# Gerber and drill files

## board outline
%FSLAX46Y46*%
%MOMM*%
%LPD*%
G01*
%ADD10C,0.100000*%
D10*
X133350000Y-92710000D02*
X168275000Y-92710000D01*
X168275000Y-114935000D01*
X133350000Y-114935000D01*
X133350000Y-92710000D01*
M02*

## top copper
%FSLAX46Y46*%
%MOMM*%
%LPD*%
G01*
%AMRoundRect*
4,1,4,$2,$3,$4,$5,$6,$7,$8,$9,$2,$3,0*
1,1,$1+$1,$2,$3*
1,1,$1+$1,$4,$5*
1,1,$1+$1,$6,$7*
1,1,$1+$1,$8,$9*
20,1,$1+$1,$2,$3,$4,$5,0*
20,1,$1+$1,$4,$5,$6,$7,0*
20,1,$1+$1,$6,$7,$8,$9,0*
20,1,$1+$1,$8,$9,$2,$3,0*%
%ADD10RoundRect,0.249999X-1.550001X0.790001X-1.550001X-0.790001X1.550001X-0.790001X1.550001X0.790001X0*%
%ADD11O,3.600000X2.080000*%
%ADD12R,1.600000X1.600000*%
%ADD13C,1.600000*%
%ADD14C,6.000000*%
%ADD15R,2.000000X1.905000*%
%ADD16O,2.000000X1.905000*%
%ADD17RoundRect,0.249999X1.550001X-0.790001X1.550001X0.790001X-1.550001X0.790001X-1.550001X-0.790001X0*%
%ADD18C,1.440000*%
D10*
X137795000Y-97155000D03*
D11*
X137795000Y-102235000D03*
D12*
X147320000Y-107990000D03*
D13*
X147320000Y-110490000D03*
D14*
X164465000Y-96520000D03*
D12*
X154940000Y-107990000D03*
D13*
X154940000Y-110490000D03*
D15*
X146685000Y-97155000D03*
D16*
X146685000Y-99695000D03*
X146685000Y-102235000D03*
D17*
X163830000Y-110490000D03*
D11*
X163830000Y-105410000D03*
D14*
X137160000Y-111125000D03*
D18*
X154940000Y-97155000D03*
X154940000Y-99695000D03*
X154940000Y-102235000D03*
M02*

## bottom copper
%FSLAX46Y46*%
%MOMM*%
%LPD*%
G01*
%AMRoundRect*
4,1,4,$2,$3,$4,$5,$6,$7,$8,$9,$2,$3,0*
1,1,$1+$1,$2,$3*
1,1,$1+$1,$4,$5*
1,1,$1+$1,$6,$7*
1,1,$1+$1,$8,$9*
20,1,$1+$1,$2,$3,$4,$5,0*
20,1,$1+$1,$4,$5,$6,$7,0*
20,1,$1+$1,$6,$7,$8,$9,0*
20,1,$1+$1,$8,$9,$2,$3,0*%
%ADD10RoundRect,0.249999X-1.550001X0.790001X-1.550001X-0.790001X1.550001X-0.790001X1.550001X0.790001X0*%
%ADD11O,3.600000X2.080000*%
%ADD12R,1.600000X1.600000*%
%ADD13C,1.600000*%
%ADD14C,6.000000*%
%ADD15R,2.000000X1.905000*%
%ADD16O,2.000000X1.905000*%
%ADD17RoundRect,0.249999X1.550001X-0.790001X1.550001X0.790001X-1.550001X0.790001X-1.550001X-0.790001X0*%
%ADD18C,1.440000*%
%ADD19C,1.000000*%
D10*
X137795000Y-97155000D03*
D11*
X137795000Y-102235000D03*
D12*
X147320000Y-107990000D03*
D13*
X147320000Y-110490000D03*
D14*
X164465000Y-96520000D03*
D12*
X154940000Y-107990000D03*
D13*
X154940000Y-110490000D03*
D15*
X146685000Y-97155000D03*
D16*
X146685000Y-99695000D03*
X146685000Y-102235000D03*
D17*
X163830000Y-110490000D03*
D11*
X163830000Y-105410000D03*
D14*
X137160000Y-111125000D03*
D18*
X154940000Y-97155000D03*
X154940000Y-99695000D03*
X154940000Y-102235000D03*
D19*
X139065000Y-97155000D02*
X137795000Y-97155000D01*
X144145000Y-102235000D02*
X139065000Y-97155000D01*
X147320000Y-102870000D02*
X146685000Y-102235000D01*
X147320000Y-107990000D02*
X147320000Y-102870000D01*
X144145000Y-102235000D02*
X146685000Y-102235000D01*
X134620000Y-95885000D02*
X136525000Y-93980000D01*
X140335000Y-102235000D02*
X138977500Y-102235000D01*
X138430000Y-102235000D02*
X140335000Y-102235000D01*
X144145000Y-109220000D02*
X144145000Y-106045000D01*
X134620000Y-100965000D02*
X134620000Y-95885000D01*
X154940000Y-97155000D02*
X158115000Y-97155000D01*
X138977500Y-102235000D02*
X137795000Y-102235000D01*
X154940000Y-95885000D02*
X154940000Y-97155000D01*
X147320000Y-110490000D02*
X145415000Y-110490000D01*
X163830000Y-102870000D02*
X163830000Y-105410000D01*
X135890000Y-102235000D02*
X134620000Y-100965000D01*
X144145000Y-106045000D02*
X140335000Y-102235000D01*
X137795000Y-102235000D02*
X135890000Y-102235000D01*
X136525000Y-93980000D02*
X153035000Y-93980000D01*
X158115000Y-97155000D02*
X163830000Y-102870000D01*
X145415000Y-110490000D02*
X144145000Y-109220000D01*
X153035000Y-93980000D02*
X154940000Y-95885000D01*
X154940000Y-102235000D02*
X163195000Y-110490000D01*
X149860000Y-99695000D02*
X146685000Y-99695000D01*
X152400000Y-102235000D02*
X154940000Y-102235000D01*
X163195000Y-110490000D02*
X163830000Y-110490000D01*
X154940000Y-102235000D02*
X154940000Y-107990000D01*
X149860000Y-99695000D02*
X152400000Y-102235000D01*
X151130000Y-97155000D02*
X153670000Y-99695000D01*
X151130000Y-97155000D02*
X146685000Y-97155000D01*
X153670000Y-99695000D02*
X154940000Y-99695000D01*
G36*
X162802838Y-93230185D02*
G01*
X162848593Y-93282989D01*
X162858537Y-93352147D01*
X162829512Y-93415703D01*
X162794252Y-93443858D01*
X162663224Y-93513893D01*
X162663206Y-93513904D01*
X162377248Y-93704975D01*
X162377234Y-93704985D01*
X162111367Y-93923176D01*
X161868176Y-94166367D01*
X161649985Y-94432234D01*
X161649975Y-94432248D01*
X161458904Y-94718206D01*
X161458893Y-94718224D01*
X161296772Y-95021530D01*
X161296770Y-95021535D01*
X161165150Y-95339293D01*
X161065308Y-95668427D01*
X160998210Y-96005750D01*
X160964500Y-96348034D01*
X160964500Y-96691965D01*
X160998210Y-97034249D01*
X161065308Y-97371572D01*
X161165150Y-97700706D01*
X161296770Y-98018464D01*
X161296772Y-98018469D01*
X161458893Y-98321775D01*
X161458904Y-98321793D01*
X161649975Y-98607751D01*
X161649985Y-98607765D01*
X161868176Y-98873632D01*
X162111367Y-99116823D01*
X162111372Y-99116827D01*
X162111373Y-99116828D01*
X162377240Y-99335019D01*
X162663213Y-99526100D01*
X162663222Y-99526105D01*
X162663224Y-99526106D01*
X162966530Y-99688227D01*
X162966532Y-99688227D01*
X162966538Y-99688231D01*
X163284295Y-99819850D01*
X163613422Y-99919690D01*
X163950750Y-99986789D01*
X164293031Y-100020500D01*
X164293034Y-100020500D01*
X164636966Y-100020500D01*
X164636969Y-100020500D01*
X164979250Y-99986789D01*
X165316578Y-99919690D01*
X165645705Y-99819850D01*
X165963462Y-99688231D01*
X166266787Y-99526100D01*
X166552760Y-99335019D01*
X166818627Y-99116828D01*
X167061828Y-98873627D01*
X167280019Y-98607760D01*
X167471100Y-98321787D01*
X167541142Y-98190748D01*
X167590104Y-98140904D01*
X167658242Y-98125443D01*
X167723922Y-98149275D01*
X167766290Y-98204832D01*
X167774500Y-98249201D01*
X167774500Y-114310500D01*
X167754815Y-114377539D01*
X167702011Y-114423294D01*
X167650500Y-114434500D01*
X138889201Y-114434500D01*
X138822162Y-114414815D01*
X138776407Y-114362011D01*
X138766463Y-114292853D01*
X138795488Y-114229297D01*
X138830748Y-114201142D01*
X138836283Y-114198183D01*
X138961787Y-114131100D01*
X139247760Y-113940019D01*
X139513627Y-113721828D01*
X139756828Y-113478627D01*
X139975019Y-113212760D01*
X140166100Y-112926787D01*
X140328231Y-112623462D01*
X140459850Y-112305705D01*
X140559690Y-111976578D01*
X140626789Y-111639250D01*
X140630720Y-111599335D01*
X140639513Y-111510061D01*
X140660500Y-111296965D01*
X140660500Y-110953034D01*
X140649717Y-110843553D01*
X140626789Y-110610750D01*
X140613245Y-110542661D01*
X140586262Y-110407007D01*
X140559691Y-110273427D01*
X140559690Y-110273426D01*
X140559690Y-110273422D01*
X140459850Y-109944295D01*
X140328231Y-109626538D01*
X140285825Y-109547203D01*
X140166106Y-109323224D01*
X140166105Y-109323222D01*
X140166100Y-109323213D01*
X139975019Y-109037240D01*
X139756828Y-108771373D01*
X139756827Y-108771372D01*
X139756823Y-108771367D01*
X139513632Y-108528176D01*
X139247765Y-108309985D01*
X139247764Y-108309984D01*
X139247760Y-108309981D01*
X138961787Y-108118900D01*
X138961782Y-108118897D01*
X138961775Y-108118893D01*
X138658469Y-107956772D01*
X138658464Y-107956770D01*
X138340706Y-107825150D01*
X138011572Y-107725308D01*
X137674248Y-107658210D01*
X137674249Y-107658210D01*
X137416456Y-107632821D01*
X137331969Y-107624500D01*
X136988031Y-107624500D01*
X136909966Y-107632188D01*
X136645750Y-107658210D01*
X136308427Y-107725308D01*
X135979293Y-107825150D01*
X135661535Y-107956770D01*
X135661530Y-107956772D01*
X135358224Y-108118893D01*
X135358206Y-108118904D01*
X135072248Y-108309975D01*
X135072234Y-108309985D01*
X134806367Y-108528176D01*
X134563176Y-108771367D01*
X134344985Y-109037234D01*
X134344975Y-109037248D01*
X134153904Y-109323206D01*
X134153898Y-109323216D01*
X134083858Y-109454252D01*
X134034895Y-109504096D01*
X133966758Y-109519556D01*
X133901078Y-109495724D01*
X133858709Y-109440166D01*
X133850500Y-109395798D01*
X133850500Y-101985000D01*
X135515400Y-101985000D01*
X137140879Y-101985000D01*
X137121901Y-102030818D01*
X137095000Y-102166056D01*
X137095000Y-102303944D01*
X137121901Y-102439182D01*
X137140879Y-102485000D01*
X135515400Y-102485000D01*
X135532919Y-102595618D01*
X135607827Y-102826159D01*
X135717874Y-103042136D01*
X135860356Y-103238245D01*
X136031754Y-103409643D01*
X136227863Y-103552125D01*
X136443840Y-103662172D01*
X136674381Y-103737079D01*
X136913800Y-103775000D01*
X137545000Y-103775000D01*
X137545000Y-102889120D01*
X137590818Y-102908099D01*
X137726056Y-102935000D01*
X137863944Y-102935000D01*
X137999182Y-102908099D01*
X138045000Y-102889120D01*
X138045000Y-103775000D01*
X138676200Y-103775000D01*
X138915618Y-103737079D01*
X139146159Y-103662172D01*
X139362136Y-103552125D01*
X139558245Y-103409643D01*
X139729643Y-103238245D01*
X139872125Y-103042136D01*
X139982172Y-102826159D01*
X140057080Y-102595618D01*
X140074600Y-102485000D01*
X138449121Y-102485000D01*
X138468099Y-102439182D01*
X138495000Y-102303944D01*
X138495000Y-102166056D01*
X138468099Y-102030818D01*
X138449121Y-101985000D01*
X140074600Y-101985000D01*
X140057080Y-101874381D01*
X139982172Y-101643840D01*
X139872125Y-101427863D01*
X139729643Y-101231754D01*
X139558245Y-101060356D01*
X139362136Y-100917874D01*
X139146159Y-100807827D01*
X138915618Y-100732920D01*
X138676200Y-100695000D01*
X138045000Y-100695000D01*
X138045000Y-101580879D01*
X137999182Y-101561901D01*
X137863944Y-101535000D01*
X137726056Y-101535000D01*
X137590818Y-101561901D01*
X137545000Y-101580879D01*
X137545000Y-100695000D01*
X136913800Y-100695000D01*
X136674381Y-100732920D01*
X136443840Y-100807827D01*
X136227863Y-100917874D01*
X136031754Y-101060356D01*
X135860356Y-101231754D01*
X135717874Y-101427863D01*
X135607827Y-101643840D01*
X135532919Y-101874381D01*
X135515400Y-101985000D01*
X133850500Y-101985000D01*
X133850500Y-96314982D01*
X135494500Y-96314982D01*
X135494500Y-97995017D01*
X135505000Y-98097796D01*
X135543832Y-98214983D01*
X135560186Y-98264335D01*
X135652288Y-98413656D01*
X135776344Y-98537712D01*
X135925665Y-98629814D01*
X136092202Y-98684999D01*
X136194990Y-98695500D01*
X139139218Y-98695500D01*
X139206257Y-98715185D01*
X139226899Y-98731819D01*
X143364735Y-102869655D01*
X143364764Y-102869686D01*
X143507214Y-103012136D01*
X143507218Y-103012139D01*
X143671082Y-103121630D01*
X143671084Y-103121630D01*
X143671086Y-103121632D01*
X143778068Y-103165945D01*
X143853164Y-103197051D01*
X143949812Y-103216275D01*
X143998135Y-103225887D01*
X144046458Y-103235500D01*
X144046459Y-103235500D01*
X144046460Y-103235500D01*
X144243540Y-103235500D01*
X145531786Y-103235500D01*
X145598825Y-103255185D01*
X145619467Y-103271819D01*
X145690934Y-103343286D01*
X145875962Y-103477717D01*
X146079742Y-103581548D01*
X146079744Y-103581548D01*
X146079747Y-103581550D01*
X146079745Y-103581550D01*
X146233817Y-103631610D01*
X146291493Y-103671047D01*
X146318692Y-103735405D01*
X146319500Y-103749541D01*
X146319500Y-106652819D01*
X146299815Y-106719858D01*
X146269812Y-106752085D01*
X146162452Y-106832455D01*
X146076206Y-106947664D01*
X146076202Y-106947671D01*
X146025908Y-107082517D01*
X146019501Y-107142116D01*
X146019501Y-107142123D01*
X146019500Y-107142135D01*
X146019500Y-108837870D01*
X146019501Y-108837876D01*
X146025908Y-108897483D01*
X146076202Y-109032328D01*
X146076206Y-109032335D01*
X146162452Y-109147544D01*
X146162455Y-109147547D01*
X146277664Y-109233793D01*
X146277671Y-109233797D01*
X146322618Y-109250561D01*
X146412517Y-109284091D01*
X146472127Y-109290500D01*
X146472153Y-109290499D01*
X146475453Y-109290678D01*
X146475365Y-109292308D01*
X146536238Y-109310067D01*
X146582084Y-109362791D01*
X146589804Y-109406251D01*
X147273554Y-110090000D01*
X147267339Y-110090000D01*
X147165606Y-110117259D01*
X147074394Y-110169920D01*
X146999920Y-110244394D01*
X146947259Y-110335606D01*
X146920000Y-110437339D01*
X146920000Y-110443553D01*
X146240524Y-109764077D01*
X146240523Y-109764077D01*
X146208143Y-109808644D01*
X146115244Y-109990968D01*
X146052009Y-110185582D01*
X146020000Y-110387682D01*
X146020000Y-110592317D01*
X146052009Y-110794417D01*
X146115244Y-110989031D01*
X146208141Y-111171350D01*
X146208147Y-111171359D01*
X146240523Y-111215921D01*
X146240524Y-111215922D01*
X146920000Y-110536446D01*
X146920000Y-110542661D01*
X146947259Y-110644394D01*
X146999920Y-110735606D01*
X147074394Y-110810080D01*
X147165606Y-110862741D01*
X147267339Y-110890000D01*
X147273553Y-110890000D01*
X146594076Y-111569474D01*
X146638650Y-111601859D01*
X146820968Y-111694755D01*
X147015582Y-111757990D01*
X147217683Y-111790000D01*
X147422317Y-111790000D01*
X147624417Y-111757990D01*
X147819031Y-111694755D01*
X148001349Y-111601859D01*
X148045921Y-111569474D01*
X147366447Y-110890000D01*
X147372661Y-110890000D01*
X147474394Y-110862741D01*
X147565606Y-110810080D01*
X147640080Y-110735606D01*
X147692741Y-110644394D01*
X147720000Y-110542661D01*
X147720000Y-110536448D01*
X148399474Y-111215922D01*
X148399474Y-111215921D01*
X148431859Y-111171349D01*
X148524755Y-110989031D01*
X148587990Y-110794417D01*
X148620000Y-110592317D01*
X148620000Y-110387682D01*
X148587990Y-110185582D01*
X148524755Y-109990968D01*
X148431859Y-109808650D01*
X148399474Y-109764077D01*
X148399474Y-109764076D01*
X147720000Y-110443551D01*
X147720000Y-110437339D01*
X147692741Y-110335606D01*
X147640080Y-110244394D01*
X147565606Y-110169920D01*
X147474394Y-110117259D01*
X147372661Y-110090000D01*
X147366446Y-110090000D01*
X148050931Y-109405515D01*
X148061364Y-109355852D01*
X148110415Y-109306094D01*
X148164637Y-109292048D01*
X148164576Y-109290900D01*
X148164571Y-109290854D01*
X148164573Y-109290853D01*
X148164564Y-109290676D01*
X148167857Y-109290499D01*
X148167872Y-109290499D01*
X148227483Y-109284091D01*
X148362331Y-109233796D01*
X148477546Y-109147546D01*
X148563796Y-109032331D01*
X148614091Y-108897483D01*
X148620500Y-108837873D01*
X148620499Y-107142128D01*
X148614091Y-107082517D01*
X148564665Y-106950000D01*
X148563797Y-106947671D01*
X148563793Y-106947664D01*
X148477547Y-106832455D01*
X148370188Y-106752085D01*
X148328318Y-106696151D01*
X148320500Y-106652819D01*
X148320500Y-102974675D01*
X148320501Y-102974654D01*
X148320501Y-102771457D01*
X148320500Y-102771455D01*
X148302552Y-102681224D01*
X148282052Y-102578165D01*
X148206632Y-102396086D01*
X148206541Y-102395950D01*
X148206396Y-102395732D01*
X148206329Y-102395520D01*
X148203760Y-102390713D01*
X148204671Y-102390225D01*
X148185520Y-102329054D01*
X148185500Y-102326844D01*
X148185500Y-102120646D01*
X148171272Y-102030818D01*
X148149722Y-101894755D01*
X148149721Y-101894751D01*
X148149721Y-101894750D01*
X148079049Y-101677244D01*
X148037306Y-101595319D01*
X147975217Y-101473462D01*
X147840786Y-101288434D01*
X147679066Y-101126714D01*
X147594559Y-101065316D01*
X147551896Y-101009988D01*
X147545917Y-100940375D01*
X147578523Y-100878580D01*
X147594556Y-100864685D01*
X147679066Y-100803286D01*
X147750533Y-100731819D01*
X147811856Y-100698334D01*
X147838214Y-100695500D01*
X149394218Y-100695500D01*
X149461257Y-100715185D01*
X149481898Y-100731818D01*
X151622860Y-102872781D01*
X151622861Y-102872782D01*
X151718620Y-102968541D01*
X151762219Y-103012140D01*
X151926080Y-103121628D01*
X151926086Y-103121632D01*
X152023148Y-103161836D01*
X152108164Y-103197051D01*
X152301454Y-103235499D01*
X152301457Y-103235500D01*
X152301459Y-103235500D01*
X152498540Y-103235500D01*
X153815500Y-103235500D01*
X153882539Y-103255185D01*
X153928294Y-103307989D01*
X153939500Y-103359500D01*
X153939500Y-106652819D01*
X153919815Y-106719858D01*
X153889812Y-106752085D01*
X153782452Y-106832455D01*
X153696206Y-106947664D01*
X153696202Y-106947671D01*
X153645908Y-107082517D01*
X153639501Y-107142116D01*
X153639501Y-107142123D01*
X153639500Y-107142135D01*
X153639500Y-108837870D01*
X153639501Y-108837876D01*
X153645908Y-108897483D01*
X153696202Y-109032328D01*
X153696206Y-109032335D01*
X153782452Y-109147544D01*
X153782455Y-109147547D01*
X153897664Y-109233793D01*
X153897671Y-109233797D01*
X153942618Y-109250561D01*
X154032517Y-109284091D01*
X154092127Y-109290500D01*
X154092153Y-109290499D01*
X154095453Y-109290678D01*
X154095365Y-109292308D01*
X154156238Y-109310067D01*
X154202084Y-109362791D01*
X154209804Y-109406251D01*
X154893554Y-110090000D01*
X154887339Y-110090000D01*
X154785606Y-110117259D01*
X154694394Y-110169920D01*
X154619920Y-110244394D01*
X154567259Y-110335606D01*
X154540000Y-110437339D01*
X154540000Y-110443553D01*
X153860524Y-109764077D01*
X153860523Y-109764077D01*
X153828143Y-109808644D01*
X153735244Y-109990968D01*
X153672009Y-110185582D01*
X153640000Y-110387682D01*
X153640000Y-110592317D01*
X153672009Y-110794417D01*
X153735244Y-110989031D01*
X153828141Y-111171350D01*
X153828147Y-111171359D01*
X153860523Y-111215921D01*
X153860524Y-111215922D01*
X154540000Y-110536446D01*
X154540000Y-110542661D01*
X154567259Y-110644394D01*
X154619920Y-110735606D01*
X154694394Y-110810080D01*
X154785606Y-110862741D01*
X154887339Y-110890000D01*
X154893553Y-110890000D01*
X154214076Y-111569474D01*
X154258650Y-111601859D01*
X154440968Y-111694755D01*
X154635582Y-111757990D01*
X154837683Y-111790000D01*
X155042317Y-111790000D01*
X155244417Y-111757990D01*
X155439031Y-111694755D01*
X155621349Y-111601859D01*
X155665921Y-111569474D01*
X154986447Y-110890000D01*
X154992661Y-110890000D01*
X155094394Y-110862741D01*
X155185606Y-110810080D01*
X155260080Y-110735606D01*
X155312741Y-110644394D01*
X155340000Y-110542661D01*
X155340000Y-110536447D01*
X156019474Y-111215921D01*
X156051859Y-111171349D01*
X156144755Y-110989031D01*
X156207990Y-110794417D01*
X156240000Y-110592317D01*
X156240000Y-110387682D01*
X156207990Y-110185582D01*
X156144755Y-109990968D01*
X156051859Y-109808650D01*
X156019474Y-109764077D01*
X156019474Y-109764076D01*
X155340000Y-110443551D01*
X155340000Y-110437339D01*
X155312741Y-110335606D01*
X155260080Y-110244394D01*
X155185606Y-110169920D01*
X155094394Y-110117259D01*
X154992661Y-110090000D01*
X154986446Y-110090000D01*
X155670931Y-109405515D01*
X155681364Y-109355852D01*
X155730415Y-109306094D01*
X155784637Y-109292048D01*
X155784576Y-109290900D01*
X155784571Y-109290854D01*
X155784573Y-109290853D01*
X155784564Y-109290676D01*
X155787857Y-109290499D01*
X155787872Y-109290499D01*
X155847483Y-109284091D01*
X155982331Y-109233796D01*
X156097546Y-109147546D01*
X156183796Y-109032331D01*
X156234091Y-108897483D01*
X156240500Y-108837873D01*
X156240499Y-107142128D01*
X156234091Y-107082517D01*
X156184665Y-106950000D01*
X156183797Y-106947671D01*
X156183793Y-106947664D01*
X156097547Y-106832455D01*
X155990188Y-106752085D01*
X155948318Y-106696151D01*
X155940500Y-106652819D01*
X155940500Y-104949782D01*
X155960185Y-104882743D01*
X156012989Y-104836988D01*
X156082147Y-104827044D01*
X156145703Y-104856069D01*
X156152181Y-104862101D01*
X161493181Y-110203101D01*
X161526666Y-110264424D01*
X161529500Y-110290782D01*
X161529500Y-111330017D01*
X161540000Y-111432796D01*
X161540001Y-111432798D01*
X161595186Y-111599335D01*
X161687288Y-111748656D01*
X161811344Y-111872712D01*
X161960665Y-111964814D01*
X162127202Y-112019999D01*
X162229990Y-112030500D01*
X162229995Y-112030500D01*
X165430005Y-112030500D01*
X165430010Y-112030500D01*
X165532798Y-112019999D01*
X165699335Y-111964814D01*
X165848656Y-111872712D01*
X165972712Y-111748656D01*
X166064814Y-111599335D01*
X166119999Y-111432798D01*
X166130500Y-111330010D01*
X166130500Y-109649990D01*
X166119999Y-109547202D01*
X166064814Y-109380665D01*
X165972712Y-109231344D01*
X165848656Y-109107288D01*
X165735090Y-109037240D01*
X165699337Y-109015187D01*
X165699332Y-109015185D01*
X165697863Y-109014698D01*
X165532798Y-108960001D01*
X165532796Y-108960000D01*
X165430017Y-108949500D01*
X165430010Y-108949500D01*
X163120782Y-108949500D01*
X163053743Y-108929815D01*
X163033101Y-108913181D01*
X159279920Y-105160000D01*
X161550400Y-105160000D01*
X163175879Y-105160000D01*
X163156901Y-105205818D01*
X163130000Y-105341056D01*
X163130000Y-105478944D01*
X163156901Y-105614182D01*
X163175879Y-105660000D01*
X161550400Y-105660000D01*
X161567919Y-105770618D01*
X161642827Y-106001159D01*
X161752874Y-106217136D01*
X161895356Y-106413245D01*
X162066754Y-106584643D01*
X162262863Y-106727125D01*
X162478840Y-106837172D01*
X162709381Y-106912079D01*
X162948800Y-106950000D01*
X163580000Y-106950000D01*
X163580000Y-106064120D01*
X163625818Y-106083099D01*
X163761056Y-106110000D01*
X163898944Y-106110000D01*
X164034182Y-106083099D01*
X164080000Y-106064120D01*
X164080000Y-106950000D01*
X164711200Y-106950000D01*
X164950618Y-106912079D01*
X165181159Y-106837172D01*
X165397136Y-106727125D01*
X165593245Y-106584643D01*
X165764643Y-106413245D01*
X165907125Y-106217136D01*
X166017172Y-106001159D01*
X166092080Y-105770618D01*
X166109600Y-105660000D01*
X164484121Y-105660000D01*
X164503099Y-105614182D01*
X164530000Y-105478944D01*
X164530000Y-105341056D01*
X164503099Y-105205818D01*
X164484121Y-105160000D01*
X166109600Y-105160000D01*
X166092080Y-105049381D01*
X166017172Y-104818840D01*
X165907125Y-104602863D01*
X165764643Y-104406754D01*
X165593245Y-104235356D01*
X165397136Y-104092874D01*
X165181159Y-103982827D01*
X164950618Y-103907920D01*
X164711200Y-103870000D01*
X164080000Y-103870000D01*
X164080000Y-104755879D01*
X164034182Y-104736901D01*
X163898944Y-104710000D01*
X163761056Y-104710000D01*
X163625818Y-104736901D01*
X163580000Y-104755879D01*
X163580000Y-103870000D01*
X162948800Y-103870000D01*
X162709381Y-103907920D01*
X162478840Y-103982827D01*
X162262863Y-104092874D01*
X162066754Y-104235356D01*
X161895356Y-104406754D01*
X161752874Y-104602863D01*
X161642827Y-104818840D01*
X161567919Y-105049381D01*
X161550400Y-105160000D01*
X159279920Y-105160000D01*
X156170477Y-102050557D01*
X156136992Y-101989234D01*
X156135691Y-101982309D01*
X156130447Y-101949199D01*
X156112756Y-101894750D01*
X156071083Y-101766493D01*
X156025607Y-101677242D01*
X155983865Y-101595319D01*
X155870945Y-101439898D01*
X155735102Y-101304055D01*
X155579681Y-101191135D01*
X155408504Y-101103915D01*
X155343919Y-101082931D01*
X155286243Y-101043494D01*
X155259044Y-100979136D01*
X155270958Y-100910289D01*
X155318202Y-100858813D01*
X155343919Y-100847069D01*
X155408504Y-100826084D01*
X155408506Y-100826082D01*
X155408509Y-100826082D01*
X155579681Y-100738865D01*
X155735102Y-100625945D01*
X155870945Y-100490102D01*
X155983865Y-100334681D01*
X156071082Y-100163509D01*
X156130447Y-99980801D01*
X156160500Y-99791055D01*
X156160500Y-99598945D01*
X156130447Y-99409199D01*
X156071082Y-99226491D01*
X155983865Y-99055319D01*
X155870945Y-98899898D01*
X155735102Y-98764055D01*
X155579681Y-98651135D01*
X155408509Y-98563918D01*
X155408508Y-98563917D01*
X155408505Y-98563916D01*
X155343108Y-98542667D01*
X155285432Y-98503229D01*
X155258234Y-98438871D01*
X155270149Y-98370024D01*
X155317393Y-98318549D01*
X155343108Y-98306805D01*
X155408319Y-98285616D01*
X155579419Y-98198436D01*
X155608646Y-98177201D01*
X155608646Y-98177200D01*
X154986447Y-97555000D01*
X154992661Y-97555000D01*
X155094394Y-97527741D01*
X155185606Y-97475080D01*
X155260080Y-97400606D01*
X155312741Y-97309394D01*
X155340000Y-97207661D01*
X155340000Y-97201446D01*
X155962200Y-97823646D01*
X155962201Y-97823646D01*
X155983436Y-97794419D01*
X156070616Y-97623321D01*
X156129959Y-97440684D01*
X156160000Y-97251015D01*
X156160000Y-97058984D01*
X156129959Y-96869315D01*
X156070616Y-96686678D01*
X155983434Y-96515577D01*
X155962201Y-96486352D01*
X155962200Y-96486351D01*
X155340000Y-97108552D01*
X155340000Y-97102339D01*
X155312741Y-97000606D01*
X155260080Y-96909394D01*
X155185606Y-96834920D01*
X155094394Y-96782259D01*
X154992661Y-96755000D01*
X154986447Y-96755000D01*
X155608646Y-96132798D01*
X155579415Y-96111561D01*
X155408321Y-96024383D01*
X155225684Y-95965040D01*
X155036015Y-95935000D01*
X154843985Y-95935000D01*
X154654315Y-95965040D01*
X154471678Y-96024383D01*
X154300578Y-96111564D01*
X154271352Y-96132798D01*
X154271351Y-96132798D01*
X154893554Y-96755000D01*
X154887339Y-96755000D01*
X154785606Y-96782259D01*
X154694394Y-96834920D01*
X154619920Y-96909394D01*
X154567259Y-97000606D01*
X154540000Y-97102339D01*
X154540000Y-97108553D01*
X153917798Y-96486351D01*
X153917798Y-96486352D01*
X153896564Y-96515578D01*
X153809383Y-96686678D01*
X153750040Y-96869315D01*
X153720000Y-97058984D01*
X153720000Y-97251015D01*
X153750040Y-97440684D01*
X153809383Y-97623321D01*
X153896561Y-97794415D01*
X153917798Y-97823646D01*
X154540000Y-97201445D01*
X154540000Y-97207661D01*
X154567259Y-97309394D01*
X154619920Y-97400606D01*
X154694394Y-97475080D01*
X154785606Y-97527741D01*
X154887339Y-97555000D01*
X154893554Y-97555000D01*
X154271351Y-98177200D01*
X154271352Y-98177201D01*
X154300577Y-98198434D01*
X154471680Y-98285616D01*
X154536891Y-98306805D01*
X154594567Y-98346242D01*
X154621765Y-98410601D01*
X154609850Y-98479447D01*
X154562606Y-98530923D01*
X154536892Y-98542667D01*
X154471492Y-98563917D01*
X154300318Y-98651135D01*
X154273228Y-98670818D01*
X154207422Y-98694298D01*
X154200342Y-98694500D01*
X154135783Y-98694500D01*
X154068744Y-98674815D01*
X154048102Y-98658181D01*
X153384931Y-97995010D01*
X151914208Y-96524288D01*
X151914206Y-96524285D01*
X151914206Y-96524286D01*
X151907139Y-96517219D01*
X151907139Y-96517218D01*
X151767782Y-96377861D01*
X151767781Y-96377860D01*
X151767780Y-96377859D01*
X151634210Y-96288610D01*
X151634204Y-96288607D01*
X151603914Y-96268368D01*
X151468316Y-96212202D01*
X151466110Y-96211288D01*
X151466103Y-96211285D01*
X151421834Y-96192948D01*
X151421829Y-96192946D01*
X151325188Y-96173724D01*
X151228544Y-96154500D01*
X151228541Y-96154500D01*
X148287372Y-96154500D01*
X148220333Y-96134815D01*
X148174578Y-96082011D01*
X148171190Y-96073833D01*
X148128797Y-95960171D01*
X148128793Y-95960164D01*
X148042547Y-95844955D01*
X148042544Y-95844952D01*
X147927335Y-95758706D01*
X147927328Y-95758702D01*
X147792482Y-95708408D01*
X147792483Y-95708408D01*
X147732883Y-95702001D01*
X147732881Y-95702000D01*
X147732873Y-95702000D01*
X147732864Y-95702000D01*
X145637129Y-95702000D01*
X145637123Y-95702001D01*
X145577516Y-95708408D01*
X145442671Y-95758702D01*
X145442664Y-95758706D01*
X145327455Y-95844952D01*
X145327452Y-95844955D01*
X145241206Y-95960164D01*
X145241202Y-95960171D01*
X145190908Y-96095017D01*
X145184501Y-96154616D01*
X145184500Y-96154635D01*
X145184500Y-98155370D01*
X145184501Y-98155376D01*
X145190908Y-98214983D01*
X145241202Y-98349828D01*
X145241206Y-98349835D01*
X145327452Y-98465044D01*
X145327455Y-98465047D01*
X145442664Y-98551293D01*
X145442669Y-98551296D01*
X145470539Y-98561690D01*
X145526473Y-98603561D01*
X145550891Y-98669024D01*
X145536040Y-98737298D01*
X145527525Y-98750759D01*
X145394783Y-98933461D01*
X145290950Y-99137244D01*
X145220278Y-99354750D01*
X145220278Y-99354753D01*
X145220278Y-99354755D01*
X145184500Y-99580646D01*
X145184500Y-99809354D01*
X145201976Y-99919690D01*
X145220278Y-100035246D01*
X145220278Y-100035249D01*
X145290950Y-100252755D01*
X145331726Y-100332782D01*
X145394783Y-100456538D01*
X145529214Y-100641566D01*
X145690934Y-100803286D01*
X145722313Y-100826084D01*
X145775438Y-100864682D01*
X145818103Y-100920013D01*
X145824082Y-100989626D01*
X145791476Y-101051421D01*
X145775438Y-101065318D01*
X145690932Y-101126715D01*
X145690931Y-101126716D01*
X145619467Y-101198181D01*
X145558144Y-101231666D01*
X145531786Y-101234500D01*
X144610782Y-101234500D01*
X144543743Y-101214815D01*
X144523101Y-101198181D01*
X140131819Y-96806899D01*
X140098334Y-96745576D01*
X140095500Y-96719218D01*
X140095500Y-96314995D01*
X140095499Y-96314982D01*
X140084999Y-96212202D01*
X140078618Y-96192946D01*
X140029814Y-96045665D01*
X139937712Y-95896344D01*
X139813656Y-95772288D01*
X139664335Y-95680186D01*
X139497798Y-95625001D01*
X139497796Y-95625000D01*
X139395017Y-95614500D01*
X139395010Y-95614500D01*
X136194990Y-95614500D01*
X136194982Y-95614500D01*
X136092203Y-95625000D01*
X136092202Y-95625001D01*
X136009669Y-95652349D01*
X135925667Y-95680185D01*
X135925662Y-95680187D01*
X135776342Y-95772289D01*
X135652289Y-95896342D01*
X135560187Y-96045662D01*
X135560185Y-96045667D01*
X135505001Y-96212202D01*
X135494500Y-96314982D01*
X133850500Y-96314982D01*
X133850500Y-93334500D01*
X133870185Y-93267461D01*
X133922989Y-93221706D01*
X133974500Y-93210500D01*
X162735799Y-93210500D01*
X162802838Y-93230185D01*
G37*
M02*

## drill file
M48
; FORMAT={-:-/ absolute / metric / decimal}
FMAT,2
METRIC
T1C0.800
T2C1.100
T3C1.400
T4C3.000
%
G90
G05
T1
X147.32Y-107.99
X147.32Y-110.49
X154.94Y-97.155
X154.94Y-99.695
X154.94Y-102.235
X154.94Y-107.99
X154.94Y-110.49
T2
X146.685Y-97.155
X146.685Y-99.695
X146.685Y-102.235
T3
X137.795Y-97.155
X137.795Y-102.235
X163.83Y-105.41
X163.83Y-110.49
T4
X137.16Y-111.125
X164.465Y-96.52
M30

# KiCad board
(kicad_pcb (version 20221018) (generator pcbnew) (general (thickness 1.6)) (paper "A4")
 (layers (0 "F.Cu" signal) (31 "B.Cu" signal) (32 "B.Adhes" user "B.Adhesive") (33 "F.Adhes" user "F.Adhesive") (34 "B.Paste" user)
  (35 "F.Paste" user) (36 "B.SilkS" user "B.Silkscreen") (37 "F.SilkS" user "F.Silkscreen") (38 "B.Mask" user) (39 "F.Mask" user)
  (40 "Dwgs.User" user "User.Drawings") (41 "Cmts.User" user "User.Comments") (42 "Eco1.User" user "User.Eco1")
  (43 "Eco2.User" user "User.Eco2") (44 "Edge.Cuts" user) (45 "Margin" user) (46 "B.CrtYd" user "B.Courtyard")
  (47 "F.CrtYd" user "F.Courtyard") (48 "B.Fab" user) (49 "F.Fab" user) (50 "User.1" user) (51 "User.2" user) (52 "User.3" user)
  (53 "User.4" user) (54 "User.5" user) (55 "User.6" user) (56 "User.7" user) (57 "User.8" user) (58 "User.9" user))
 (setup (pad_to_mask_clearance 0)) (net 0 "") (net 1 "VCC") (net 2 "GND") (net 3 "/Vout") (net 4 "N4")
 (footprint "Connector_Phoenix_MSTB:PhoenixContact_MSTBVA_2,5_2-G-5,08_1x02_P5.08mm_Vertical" (layer "F.Cu") (at 137.795 97.155 -90)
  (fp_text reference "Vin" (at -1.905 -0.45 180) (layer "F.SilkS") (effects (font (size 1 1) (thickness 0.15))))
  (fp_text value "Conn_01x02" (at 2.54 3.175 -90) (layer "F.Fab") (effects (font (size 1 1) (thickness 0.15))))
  (pad "1" thru_hole roundrect (at 0 0 270) (size 2.08 3.6) (drill 1.4) (layers "*.Cu" "*.Mask") (roundrect_rratio 0.1201918269)
   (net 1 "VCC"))
  (pad "2" thru_hole oval (at 5.08 0 270) (size 2.08 3.6) (drill 1.4) (layers "*.Cu" "*.Mask") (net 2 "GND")))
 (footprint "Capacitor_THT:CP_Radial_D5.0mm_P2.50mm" (layer "F.Cu") (at 147.32 107.99 -90)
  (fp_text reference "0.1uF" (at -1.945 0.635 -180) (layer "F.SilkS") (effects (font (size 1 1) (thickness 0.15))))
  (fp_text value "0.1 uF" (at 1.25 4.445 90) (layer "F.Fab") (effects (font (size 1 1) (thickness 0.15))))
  (pad "1" thru_hole rect (at 0 0 270) (size 1.6 1.6) (drill 0.8) (layers "*.Cu" "*.Mask") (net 1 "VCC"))
  (pad "2" thru_hole circle (at 2.5 0 270) (size 1.6 1.6) (drill 0.8) (layers "*.Cu" "*.Mask") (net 2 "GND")))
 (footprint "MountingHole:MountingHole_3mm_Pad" (layer "F.Cu") (at 164.465 96.52)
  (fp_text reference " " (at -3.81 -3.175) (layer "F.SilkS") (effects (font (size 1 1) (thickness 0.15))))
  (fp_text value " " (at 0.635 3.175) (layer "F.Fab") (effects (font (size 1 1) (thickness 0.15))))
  (pad "1" thru_hole circle (at 0 0) (size 6 6) (drill 3) (layers "*.Cu" "*.Mask")))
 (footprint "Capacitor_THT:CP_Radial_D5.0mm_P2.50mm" (layer "F.Cu") (at 154.94 107.99 -90)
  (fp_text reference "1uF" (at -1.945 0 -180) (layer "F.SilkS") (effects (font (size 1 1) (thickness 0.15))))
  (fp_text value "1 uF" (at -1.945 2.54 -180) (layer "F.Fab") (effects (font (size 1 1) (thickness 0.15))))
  (pad "1" thru_hole rect (at 0 0 270) (size 1.6 1.6) (drill 0.8) (layers "*.Cu" "*.Mask") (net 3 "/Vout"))
  (pad "2" thru_hole circle (at 2.5 0 270) (size 1.6 1.6) (drill 0.8) (layers "*.Cu" "*.Mask") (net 2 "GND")))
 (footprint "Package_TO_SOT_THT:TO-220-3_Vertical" (layer "F.Cu") (at 146.685 97.155 -90)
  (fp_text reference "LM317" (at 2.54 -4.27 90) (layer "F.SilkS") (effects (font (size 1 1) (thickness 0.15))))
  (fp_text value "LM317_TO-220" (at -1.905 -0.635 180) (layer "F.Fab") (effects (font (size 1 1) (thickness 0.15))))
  (pad "1" thru_hole rect (at 0 0 270) (size 1.905 2) (drill 1.1) (layers "*.Cu" "*.Mask") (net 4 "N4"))
  (pad "2" thru_hole oval (at 2.54 0 270) (size 1.905 2) (drill 1.1) (layers "*.Cu" "*.Mask") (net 3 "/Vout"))
  (pad "3" thru_hole oval (at 5.08 0 270) (size 1.905 2) (drill 1.1) (layers "*.Cu" "*.Mask") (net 1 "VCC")))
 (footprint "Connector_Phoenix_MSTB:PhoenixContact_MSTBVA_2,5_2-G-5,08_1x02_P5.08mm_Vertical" (layer "F.Cu") (at 163.83 110.49 90)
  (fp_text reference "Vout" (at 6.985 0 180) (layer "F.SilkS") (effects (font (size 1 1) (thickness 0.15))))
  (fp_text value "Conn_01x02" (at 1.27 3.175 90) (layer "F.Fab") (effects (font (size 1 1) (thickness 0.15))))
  (pad "1" thru_hole roundrect (at 0 0 90) (size 2.08 3.6) (drill 1.4) (layers "*.Cu" "*.Mask") (roundrect_rratio 0.1201918269)
   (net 3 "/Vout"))
  (pad "2" thru_hole oval (at 5.08 0 90) (size 2.08 3.6) (drill 1.4) (layers "*.Cu" "*.Mask") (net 2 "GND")))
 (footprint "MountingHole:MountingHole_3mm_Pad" (layer "F.Cu") (at 137.16 111.125)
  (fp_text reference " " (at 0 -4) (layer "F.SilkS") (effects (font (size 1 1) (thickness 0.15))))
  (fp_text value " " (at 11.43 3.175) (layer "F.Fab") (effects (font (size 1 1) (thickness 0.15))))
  (pad "1" thru_hole circle (at 0 0) (size 6 6) (drill 3) (layers "*.Cu" "*.Mask")))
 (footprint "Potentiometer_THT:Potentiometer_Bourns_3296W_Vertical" (layer "F.Cu") (at 154.94 97.155 90)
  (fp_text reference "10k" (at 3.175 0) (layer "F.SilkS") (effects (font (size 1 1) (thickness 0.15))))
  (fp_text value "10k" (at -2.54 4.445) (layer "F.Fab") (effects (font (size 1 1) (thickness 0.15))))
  (pad "1" thru_hole circle (at 0 0 90) (size 1.44 1.44) (drill 0.8) (layers "*.Cu" "*.Mask") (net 2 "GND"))
  (pad "2" thru_hole circle (at -2.54 0 90) (size 1.44 1.44) (drill 0.8) (layers "*.Cu" "*.Mask") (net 4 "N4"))
  (pad "3" thru_hole circle (at -5.08 0 90) (size 1.44 1.44) (drill 0.8) (layers "*.Cu" "*.Mask") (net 3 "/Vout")))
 (gr_rect (start 133.35 92.71) (end 168.275 114.935) (stroke (width 0.1) (type default)) (fill none) (layer "Edge.Cuts"))
 (segment (start 139.065 97.155) (end 137.795 97.155) (width 1) (layer "B.Cu") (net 1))
 (segment (start 144.145 102.235) (end 139.065 97.155) (width 1) (layer "B.Cu") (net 1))
 (segment (start 147.32 102.87) (end 146.685 102.235) (width 1) (layer "B.Cu") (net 1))
 (segment (start 147.32 107.99) (end 147.32 102.87) (width 1) (layer "B.Cu") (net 1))
 (segment (start 144.145 102.235) (end 146.685 102.235) (width 1) (layer "B.Cu") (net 1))
 (segment (start 134.62 95.885) (end 136.525 93.98) (width 1) (layer "B.Cu") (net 2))
 (segment (start 140.335 102.235) (end 138.9775 102.235) (width 1) (layer "B.Cu") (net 2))
 (segment (start 138.43 102.235) (end 140.335 102.235) (width 1) (layer "B.Cu") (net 2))
 (segment (start 144.145 109.22) (end 144.145 106.045) (width 1) (layer "B.Cu") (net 2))
 (segment (start 134.62 100.965) (end 134.62 95.885) (width 1) (layer "B.Cu") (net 2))
 (segment (start 154.94 97.155) (end 158.115 97.155) (width 1) (layer "B.Cu") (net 2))
 (segment (start 138.9775 102.235) (end 137.795 102.235) (width 1) (layer "B.Cu") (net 2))
 (segment (start 154.94 95.885) (end 154.94 97.155) (width 1) (layer "B.Cu") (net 2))
 (segment (start 147.32 110.49) (end 145.415 110.49) (width 1) (layer "B.Cu") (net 2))
 (segment (start 163.83 102.87) (end 163.83 105.41) (width 1) (layer "B.Cu") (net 2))
 (segment (start 135.89 102.235) (end 134.62 100.965) (width 1) (layer "B.Cu") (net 2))
 (segment (start 144.145 106.045) (end 140.335 102.235) (width 1) (layer "B.Cu") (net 2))
 (segment (start 137.795 102.235) (end 135.89 102.235) (width 1) (layer "B.Cu") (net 2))
 (segment (start 136.525 93.98) (end 153.035 93.98) (width 1) (layer "B.Cu") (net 2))
 (segment (start 158.115 97.155) (end 163.83 102.87) (width 1) (layer "B.Cu") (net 2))
 (segment (start 145.415 110.49) (end 144.145 109.22) (width 1) (layer "B.Cu") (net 2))
 (segment (start 153.035 93.98) (end 154.94 95.885) (width 1) (layer "B.Cu") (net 2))
 (segment (start 154.94 102.235) (end 163.195 110.49) (width 1) (layer "B.Cu") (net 3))
 (segment (start 149.86 99.695) (end 146.685 99.695) (width 1) (layer "B.Cu") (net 3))
 (segment (start 152.4 102.235) (end 154.94 102.235) (width 1) (layer "B.Cu") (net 3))
 (segment (start 163.195 110.49) (end 163.83 110.49) (width 1) (layer "B.Cu") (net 3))
 (segment (start 154.94 102.235) (end 154.94 107.99) (width 1) (layer "B.Cu") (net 3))
 (segment (start 149.86 99.695) (end 152.4 102.235) (width 1) (layer "B.Cu") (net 3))
 (segment (start 151.13 97.155) (end 153.67 99.695) (width 1) (layer "B.Cu") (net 4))
 (segment (start 151.13 97.155) (end 146.685 97.155) (width 1) (layer "B.Cu") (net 4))
 (segment (start 153.67 99.695) (end 154.94 99.695) (width 1) (layer "B.Cu") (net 4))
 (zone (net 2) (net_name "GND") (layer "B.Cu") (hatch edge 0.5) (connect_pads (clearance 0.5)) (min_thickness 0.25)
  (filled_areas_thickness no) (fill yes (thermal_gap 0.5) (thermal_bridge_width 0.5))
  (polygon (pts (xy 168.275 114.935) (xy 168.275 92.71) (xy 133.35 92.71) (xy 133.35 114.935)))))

